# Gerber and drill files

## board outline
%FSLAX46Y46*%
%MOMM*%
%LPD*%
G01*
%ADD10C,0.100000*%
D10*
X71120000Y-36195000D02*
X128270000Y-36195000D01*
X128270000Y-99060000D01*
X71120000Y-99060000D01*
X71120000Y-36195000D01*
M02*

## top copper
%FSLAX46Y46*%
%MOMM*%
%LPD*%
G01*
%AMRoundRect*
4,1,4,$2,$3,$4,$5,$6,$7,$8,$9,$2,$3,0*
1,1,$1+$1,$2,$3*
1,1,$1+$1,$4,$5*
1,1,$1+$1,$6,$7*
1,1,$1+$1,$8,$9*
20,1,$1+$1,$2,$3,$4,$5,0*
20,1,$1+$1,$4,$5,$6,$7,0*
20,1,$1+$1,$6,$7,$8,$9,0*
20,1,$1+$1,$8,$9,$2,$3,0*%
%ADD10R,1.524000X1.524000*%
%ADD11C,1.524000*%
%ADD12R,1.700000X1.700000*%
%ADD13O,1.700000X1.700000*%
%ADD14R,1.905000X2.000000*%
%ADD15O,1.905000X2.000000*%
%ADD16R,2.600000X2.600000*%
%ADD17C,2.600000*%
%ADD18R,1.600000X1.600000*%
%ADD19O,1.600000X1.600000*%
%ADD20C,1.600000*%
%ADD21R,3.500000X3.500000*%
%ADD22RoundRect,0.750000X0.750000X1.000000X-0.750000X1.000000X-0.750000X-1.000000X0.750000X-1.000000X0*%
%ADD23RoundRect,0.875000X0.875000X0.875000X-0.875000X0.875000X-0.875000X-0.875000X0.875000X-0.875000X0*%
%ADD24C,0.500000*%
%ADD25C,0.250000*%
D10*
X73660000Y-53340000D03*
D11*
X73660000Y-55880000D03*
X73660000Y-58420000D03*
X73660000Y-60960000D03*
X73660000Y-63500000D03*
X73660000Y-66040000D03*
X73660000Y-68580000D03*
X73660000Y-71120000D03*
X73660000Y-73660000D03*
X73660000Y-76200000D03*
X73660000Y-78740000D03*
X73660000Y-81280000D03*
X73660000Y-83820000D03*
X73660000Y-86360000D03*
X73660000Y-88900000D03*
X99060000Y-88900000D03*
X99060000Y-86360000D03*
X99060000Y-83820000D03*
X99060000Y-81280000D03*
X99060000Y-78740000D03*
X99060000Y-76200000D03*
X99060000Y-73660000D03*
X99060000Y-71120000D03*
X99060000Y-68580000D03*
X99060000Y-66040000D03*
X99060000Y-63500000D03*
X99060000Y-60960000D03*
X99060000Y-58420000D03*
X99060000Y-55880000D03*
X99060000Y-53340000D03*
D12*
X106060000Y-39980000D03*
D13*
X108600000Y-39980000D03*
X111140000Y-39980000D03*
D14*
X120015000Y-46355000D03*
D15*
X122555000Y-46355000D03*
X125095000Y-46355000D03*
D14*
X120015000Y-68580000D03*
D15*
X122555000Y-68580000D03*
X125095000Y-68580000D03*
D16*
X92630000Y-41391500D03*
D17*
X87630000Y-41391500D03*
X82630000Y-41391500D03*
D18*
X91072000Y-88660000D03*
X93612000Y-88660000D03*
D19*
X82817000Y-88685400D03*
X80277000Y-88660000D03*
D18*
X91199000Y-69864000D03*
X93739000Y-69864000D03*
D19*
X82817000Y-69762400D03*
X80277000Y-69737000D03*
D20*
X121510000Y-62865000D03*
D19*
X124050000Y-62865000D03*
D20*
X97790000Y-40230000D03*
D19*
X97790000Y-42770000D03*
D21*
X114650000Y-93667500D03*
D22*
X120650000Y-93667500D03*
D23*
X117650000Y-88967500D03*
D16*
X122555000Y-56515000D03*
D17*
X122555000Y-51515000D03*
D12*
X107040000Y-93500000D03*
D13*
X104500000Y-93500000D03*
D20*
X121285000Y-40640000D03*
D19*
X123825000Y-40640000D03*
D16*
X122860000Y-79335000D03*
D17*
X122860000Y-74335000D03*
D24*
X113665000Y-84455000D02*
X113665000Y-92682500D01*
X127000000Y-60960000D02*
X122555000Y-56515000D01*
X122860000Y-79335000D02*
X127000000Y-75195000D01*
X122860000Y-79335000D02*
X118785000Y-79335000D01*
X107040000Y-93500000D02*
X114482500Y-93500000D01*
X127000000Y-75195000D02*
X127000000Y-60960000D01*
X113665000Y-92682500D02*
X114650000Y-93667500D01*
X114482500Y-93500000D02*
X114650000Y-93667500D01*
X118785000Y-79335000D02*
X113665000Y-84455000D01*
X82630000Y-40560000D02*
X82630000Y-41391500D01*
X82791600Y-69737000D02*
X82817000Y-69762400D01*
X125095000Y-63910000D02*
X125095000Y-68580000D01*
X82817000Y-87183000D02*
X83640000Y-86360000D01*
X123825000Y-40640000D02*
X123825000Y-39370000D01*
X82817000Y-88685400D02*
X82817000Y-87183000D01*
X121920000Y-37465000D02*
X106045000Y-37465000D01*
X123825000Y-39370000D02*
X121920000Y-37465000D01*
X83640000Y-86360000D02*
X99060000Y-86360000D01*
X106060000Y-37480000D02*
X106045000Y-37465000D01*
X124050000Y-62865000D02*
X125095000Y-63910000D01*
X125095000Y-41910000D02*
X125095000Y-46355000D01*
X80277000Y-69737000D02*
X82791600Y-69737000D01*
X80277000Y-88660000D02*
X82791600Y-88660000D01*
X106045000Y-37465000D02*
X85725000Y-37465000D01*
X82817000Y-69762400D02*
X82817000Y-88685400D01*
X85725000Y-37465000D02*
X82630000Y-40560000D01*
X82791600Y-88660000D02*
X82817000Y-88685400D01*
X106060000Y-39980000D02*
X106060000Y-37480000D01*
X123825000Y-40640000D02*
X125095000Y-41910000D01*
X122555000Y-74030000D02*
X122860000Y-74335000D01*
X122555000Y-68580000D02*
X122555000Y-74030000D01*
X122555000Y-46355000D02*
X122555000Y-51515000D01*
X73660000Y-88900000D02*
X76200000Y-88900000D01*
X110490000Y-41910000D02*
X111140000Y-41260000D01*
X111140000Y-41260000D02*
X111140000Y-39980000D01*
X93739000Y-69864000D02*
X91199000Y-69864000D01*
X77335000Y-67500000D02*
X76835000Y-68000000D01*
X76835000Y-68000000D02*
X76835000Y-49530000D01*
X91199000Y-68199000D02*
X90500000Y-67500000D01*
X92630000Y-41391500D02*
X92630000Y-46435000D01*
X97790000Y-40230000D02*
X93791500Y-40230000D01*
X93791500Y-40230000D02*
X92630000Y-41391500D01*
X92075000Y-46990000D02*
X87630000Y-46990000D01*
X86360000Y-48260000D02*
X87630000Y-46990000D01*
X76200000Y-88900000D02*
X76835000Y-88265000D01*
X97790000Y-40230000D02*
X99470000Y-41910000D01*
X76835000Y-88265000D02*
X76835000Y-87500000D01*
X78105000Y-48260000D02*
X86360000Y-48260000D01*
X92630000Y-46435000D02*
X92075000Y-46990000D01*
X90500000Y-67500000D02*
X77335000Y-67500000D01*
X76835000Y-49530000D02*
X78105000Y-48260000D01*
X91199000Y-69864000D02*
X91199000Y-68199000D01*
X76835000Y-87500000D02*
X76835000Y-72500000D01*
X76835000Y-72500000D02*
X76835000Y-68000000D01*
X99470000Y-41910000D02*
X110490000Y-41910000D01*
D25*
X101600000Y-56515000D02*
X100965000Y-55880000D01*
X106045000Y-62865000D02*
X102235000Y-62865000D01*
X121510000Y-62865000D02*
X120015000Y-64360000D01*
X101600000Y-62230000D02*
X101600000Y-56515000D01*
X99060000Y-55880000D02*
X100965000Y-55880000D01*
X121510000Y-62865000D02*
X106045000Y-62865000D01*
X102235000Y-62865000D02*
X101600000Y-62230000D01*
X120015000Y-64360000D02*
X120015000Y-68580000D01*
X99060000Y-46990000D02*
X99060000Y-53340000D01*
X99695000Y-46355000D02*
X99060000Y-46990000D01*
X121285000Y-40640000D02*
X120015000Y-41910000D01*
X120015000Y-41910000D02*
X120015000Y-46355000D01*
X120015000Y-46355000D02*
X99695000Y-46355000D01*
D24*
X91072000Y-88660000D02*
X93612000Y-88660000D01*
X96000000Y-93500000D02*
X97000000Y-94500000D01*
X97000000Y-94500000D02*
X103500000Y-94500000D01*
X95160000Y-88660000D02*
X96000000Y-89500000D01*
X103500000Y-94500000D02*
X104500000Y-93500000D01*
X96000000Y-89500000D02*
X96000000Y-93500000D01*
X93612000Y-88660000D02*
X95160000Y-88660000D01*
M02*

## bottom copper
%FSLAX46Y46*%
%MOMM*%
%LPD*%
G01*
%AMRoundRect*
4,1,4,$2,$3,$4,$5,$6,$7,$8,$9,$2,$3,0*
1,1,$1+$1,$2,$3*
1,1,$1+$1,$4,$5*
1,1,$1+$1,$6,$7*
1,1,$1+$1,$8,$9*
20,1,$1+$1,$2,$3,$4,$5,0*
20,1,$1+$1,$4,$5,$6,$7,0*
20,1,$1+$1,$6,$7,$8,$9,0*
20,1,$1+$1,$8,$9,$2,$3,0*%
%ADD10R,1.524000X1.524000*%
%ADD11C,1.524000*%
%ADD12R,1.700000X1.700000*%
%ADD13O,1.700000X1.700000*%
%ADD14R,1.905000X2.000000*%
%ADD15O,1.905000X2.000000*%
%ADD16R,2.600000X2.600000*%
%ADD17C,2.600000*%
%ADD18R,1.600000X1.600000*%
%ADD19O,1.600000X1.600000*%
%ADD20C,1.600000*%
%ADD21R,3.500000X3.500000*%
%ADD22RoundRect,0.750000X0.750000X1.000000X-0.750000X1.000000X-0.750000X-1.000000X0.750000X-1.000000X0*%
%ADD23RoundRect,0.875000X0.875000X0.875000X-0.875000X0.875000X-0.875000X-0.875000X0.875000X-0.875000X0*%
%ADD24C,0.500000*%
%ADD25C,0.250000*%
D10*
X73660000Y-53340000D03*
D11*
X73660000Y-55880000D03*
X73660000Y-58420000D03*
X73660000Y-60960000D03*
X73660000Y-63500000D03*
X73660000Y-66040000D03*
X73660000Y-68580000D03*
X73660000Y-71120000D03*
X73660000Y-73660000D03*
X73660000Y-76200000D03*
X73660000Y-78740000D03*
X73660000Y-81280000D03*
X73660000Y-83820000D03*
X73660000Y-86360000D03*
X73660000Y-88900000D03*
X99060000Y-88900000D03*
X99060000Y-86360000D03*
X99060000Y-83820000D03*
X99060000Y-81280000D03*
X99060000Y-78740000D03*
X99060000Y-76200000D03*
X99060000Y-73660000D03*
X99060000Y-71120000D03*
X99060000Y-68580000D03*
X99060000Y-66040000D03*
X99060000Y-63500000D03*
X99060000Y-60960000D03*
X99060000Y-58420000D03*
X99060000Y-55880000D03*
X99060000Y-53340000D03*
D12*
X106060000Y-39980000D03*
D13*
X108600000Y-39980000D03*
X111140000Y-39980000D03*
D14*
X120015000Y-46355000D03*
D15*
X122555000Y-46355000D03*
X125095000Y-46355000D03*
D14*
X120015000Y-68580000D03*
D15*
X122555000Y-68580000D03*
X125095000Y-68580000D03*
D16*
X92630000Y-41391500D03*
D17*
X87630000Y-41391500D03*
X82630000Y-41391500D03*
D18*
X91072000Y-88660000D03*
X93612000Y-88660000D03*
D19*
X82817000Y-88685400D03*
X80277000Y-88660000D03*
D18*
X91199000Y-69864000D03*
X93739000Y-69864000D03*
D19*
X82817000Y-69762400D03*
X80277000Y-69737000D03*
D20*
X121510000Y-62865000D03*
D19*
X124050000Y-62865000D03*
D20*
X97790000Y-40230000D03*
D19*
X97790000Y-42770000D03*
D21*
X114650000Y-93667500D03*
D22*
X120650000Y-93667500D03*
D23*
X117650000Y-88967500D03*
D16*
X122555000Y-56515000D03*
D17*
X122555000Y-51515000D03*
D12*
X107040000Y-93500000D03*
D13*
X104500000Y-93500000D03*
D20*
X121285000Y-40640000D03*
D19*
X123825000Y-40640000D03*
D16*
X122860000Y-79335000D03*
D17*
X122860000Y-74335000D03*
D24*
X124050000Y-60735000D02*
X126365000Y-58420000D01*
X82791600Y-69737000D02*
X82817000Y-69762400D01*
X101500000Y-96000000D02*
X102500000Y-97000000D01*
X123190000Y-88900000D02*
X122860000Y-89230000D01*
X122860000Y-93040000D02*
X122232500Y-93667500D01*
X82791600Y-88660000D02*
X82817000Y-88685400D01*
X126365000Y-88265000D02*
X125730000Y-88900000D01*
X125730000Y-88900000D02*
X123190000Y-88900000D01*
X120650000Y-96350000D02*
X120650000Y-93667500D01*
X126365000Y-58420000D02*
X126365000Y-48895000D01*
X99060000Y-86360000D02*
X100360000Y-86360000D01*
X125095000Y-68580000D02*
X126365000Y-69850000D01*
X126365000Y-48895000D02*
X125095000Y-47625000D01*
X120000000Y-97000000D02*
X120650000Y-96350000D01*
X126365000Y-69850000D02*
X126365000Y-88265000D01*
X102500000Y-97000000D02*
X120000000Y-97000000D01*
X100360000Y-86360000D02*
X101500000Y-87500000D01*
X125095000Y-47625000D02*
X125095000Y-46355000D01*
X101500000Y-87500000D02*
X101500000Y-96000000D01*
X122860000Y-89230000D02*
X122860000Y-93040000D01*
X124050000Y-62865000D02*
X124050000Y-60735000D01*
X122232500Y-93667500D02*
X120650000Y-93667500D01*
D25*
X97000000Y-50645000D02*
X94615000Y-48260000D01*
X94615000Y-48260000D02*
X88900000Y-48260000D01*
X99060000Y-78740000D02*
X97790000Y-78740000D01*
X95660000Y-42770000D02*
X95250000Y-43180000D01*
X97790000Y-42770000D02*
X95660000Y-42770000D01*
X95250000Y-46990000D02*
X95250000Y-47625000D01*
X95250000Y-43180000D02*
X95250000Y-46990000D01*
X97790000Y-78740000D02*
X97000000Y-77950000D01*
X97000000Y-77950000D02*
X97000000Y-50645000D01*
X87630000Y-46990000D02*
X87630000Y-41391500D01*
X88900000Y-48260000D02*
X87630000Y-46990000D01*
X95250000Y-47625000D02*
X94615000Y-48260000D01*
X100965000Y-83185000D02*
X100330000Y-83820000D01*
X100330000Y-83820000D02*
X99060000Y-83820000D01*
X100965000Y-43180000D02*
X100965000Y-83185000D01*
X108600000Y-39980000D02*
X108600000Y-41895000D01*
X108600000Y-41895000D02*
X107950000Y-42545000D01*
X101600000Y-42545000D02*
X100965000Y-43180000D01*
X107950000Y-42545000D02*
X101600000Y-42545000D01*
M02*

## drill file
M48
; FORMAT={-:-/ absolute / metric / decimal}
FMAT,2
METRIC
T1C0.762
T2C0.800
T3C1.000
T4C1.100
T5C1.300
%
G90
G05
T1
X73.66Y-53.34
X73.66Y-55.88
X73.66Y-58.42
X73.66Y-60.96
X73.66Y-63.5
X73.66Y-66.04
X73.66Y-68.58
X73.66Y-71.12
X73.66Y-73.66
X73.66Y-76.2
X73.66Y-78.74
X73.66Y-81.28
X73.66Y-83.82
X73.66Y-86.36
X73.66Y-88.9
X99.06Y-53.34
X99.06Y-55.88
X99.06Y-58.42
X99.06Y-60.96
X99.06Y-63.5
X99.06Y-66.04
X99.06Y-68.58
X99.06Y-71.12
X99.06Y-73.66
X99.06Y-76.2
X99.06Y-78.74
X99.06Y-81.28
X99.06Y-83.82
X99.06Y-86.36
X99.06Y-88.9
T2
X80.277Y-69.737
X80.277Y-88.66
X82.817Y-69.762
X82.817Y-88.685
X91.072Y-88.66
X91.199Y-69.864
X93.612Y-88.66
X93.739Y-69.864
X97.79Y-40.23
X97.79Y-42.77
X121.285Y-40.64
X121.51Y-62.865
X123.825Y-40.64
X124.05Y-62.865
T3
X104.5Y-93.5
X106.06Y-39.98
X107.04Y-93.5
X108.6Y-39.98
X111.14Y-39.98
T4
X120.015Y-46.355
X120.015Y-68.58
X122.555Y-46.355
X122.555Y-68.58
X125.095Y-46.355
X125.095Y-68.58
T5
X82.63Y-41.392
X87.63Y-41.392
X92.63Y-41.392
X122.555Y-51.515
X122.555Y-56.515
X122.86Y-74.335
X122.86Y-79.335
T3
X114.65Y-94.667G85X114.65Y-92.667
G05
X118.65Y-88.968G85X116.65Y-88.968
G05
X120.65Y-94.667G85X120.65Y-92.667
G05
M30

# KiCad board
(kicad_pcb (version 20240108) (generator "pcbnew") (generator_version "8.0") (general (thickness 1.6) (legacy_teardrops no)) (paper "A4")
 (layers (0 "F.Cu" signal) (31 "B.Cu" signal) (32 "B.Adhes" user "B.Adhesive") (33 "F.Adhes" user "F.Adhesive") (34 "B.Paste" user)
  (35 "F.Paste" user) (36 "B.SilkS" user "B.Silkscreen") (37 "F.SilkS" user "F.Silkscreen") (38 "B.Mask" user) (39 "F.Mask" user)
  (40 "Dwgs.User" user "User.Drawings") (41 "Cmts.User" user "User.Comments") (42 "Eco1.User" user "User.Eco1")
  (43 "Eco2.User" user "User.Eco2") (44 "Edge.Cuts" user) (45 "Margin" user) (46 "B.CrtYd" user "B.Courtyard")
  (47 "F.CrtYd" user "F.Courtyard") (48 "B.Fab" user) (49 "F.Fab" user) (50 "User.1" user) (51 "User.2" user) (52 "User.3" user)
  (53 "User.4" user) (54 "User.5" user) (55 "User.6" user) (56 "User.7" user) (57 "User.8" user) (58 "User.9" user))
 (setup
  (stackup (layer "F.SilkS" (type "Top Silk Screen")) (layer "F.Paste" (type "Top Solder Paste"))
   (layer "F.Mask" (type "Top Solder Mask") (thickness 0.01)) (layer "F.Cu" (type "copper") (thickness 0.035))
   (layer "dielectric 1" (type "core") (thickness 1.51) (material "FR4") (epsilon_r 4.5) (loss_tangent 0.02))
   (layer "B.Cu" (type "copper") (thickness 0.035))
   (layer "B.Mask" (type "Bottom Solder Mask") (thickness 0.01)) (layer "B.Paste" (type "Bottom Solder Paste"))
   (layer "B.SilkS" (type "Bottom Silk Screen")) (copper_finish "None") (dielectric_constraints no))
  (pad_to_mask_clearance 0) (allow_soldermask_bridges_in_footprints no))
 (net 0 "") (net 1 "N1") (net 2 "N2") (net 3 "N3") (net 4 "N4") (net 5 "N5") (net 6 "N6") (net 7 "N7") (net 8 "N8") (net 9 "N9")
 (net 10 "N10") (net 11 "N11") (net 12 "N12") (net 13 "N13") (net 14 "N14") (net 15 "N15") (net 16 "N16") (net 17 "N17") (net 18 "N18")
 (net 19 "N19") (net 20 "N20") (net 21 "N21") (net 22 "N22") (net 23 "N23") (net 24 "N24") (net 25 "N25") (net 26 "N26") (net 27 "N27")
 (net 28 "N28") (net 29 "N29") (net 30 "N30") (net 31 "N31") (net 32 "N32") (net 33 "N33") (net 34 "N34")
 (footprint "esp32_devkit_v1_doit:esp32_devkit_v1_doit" (layer "F.Cu") (at 86.36 53.34)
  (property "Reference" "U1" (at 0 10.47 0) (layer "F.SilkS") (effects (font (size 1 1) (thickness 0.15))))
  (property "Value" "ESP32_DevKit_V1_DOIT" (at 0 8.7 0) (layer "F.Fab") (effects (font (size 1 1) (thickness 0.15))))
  (pad "1" thru_hole rect (at -12.7 0) (size 1.524 1.524) (drill 0.762) (layers "*.Cu" "*.Mask") (remove_unused_layers no) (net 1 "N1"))
  (pad "2" thru_hole circle (at -12.7 2.54) (size 1.524 1.524) (drill 0.762) (layers "*.Cu" "*.Mask") (remove_unused_layers no) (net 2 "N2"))
  (pad "3" thru_hole circle (at -12.7 5.08) (size 1.524 1.524) (drill 0.762) (layers "*.Cu" "*.Mask") (remove_unused_layers no) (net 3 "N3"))
  (pad "4" thru_hole circle (at -12.7 7.62) (size 1.524 1.524) (drill 0.762) (layers "*.Cu" "*.Mask") (remove_unused_layers no) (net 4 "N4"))
  (pad "5" thru_hole circle (at -12.7 10.16) (size 1.524 1.524) (drill 0.762) (layers "*.Cu" "*.Mask") (remove_unused_layers no)
   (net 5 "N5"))
  (pad "6" thru_hole circle (at -12.7 12.7) (size 1.524 1.524) (drill 0.762) (layers "*.Cu" "*.Mask") (remove_unused_layers no) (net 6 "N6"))
  (pad "7" thru_hole circle (at -12.7 15.24) (size 1.524 1.524) (drill 0.762) (layers "*.Cu" "*.Mask") (remove_unused_layers no)
   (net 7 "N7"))
  (pad "8" thru_hole circle (at -12.7 17.78) (size 1.524 1.524) (drill 0.762) (layers "*.Cu" "*.Mask") (remove_unused_layers no)
   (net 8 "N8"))
  (pad "9" thru_hole circle (at -12.7 20.32) (size 1.524 1.524) (drill 0.762) (layers "*.Cu" "*.Mask") (remove_unused_layers no)
   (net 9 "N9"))
  (pad "10" thru_hole circle (at -12.7 22.86) (size 1.524 1.524) (drill 0.762) (layers "*.Cu" "*.Mask") (remove_unused_layers no)
   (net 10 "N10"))
  (pad "11" thru_hole circle (at -12.7 25.4) (size 1.524 1.524) (drill 0.762) (layers "*.Cu" "*.Mask") (remove_unused_layers no)
   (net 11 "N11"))
  (pad "12" thru_hole circle (at -12.7 27.94) (size 1.524 1.524) (drill 0.762) (layers "*.Cu" "*.Mask") (remove_unused_layers no)
   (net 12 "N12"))
  (pad "13" thru_hole circle (at -12.7 30.48) (size 1.524 1.524) (drill 0.762) (layers "*.Cu" "*.Mask") (remove_unused_layers no)
   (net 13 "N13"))
  (pad "14" thru_hole circle (at -12.7 33.02) (size 1.524 1.524) (drill 0.762) (layers "*.Cu" "*.Mask") (remove_unused_layers no)
   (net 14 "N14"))
  (pad "15" thru_hole circle (at -12.7 35.56) (size 1.524 1.524) (drill 0.762) (layers "*.Cu" "*.Mask") (remove_unused_layers no)
   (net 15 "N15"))
  (pad "16" thru_hole circle (at 12.7 35.56) (size 1.524 1.524) (drill 0.762) (layers "*.Cu" "*.Mask") (remove_unused_layers no)
   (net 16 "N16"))
  (pad "17" thru_hole circle (at 12.7 33.02) (size 1.524 1.524) (drill 0.762) (layers "*.Cu" "*.Mask") (remove_unused_layers no)
   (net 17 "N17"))
  (pad "18" thru_hole circle (at 12.7 30.48) (size 1.524 1.524) (drill 0.762) (layers "*.Cu" "*.Mask") (remove_unused_layers no)
   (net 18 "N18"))
  (pad "19" thru_hole circle (at 12.7 27.94) (size 1.524 1.524) (drill 0.762) (layers "*.Cu" "*.Mask") (remove_unused_layers no)
   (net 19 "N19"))
  (pad "20" thru_hole circle (at 12.7 25.4) (size 1.524 1.524) (drill 0.762) (layers "*.Cu" "*.Mask") (remove_unused_layers no)
   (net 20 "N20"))
  (pad "21" thru_hole circle (at 12.7 22.86) (size 1.524 1.524) (drill 0.762) (layers "*.Cu" "*.Mask") (remove_unused_layers no)
   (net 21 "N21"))
  (pad "22" thru_hole circle (at 12.7 20.32) (size 1.524 1.524) (drill 0.762) (layers "*.Cu" "*.Mask") (remove_unused_layers no)
   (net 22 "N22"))
  (pad "23" thru_hole circle (at 12.7 17.78) (size 1.524 1.524) (drill 0.762) (layers "*.Cu" "*.Mask") (remove_unused_layers no)
   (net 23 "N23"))
  (pad "24" thru_hole circle (at 12.7 15.24) (size 1.524 1.524) (drill 0.762) (layers "*.Cu" "*.Mask") (remove_unused_layers no)
   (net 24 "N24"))
  (pad "25" thru_hole circle (at 12.7 12.7) (size 1.524 1.524) (drill 0.762) (layers "*.Cu" "*.Mask") (remove_unused_layers no)
   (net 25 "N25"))
  (pad "26" thru_hole circle (at 12.7 10.16) (size 1.524 1.524) (drill 0.762) (layers "*.Cu" "*.Mask") (remove_unused_layers no)
   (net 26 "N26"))
  (pad "27" thru_hole circle (at 12.7 7.62) (size 1.524 1.524) (drill 0.762) (layers "*.Cu" "*.Mask") (remove_unused_layers no)
   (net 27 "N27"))
  (pad "28" thru_hole circle (at 12.7 5.08) (size 1.524 1.524) (drill 0.762) (layers "*.Cu" "*.Mask") (remove_unused_layers no)
   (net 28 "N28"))
  (pad "29" thru_hole circle (at 12.7 2.54) (size 1.524 1.524) (drill 0.762) (layers "*.Cu" "*.Mask") (remove_unused_layers no)
   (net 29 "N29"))
  (pad "30" thru_hole circle (at 12.7 0) (size 1.524 1.524) (drill 0.762) (layers "*.Cu" "*.Mask") (remove_unused_layers no) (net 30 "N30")))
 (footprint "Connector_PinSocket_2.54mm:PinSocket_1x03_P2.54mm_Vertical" (layer "F.Cu") (at 106.06 39.98 90)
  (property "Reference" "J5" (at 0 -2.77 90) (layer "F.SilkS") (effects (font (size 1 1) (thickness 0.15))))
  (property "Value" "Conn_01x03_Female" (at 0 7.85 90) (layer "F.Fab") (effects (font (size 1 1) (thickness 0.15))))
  (pad "1" thru_hole rect (at 0 0 90) (size 1.7 1.7) (drill 1) (layers "*.Cu" "*.Mask") (remove_unused_layers no) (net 17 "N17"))
  (pad "2" thru_hole oval (at 0 2.54 90) (size 1.7 1.7) (drill 1) (layers "*.Cu" "*.Mask") (remove_unused_layers no) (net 18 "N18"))
  (pad "3" thru_hole oval (at 0 5.08 90) (size 1.7 1.7) (drill 1) (layers "*.Cu" "*.Mask") (remove_unused_layers no) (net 15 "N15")))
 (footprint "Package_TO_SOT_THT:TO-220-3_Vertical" (layer "F.Cu") (at 120.015 46.355)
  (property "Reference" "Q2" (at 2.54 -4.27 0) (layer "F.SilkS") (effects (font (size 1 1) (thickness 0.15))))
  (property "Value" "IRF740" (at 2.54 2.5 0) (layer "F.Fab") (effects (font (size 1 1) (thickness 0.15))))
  (pad "1" thru_hole rect (at 0 0) (size 1.905 2) (drill 1.1) (layers "*.Cu" "*.Mask") (remove_unused_layers no) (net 30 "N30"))
  (pad "2" thru_hole oval (at 2.54 0) (size 1.905 2) (drill 1.1) (layers "*.Cu" "*.Mask") (remove_unused_layers no) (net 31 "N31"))
  (pad "3" thru_hole oval (at 5.08 0) (size 1.905 2) (drill 1.1) (layers "*.Cu" "*.Mask") (remove_unused_layers no) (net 17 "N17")))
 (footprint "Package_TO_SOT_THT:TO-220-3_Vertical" (layer "F.Cu") (at 120.015 68.58)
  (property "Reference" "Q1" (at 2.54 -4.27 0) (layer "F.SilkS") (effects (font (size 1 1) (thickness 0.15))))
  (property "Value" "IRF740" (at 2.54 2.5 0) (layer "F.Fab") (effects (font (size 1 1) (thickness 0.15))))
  (pad "1" thru_hole rect (at 0 0) (size 1.905 2) (drill 1.1) (layers "*.Cu" "*.Mask") (remove_unused_layers no) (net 29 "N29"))
  (pad "2" thru_hole oval (at 2.54 0) (size 1.905 2) (drill 1.1) (layers "*.Cu" "*.Mask") (remove_unused_layers no) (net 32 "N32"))
  (pad "3" thru_hole oval (at 5.08 0) (size 1.905 2) (drill 1.1) (layers "*.Cu" "*.Mask") (remove_unused_layers no) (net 17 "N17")))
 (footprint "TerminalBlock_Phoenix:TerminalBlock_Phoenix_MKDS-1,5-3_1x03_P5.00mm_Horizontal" (layer "F.Cu") (at 92.63 41.3915 180)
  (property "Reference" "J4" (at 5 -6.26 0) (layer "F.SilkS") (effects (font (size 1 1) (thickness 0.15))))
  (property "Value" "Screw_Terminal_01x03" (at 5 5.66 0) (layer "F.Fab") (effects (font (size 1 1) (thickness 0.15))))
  (pad "1" thru_hole rect (at 0 0 180) (size 2.6 2.6) (drill 1.3) (layers "*.Cu" "*.Mask") (remove_unused_layers no) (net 15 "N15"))
  (pad "2" thru_hole circle (at 5 0 180) (size 2.6 2.6) (drill 1.3) (layers "*.Cu" "*.Mask") (remove_unused_layers no) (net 20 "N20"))
  (pad "3" thru_hole circle (at 10 0 180) (size 2.6 2.6) (drill 1.3) (layers "*.Cu" "*.Mask") (remove_unused_layers no) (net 17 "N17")))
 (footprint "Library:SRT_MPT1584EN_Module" (layer "F.Cu") (at 86.5 78.5 90)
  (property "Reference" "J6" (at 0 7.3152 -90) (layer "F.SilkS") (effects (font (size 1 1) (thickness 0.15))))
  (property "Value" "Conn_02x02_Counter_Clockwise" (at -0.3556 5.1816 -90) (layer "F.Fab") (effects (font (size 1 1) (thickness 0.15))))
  (pad "1" thru_hole rect (at -10.16 4.572 180) (size 1.6 1.6) (drill 0.8) (layers "*.Cu" "B.Mask") (remove_unused_layers no) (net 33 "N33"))
  (pad "1" thru_hole rect (at -10.16 7.112 180) (size 1.6 1.6) (drill 0.8) (layers "*.Cu" "B.Mask") (remove_unused_layers no) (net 33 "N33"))
  (pad "2" thru_hole oval (at -10.1854 -3.683 180) (size 1.6 1.6) (drill 0.8) (layers "*.Cu" "B.Mask") (remove_unused_layers no)
   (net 17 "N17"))
  (pad "2" thru_hole oval (at -10.16 -6.223 180) (size 1.6 1.6) (drill 0.8) (layers "*.Cu" "B.Mask") (remove_unused_layers no)
   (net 17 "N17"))
  (pad "3" thru_hole rect (at 8.636 4.699 180) (size 1.6 1.6) (drill 0.8) (layers "*.Cu" "B.Mask") (remove_unused_layers no) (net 15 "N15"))
  (pad "3" thru_hole rect (at 8.636 7.239 180) (size 1.6 1.6) (drill 0.8) (layers "*.Cu" "B.Mask") (remove_unused_layers no) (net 15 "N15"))
  (pad "4" thru_hole oval (at 8.7376 -3.683 180) (size 1.6 1.6) (drill 0.8) (layers "*.Cu" "B.Mask") (remove_unused_layers no)
   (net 17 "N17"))
  (pad "4" thru_hole oval (at 8.763 -6.223 180) (size 1.6 1.6) (drill 0.8) (layers "*.Cu" "B.Mask") (remove_unused_layers no) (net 17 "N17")))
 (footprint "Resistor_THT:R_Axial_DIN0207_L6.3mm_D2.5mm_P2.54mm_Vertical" (layer "F.Cu") (at 121.51 62.865)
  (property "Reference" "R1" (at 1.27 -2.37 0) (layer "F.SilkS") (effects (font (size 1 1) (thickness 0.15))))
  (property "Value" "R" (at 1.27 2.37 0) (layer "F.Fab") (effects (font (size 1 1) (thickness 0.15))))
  (pad "1" thru_hole circle (at 0 0) (size 1.6 1.6) (drill 0.8) (layers "*.Cu" "*.Mask") (remove_unused_layers no) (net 29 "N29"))
  (pad "2" thru_hole oval (at 2.54 0) (size 1.6 1.6) (drill 0.8) (layers "*.Cu" "*.Mask") (remove_unused_layers no) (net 17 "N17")))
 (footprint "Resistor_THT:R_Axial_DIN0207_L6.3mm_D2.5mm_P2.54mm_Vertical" (layer "F.Cu") (at 97.79 40.23 -90)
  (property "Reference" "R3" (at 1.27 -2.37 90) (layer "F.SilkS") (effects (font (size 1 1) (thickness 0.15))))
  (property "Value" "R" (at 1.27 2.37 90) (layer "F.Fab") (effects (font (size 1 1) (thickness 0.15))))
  (pad "1" thru_hole circle (at 0 0 270) (size 1.6 1.6) (drill 0.8) (layers "*.Cu" "*.Mask") (remove_unused_layers no) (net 15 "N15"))
  (pad "2" thru_hole oval (at 2.54 0 270) (size 1.6 1.6) (drill 0.8) (layers "*.Cu" "*.Mask") (remove_unused_layers no) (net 20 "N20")))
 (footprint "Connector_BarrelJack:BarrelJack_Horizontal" (layer "F.Cu") (at 114.65 93.6675 180)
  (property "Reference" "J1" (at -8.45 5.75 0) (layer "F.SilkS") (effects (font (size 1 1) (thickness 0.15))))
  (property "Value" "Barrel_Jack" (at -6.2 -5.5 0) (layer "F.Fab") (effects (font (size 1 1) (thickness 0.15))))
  (pad "1" thru_hole rect (at 0 0 180) (size 3.5 3.5) (drill oval 1 3) (layers "*.Cu" "*.Mask") (remove_unused_layers no) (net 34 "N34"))
  (pad "2" thru_hole roundrect (at -6 0 180) (size 3 3.5) (drill oval 1 3) (layers "*.Cu" "*.Mask") (remove_unused_layers no)
   (roundrect_rratio 0.25) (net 17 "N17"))
  (pad "3" thru_hole roundrect (at -3 4.7 180) (size 3.5 3.5) (drill oval 3 1) (layers "*.Cu" "*.Mask") (remove_unused_layers no)
   (roundrect_rratio 0.25)))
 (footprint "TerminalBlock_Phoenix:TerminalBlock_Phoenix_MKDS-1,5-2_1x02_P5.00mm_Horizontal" (layer "F.Cu") (at 122.555 56.515 90)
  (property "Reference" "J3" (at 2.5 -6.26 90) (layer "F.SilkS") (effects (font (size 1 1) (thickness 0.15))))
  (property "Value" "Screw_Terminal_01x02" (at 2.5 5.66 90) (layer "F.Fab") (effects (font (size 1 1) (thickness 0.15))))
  (pad "1" thru_hole rect (at 0 0 90) (size 2.6 2.6) (drill 1.3) (layers "*.Cu" "*.Mask") (remove_unused_layers no) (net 34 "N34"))
  (pad "2" thru_hole circle (at 5 0 90) (size 2.6 2.6) (drill 1.3) (layers "*.Cu" "*.Mask") (remove_unused_layers no) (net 31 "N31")))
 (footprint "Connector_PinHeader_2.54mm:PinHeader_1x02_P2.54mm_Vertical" (layer "F.Cu") (at 107.04 93.5 -90)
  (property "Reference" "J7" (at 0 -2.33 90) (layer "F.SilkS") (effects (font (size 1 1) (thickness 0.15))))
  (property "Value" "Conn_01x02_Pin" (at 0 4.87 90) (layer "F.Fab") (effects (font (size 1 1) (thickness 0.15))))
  (pad "1" thru_hole rect (at 0 0 270) (size 1.7 1.7) (drill 1) (layers "*.Cu" "*.Mask") (remove_unused_layers no) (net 34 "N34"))
  (pad "2" thru_hole oval (at 0 2.54 270) (size 1.7 1.7) (drill 1) (layers "*.Cu" "*.Mask") (remove_unused_layers no) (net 33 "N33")))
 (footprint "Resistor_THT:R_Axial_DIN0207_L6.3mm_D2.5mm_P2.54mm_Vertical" (layer "F.Cu") (at 121.285 40.64)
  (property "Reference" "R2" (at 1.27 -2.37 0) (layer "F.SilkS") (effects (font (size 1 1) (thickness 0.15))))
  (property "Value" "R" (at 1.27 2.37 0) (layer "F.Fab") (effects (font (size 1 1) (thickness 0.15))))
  (pad "1" thru_hole circle (at 0 0) (size 1.6 1.6) (drill 0.8) (layers "*.Cu" "*.Mask") (remove_unused_layers no) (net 30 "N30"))
  (pad "2" thru_hole oval (at 2.54 0) (size 1.6 1.6) (drill 0.8) (layers "*.Cu" "*.Mask") (remove_unused_layers no) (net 17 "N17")))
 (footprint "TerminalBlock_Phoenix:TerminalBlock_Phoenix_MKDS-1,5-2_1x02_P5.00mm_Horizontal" (layer "F.Cu") (at 122.86 79.335 90)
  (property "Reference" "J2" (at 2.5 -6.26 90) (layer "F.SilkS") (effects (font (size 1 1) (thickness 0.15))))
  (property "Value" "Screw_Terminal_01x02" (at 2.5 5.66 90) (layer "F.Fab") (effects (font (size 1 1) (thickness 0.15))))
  (pad "1" thru_hole rect (at 0 0 90) (size 2.6 2.6) (drill 1.3) (layers "*.Cu" "*.Mask") (remove_unused_layers no) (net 34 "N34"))
  (pad "2" thru_hole circle (at 5 0 90) (size 2.6 2.6) (drill 1.3) (layers "*.Cu" "*.Mask") (remove_unused_layers no) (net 32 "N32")))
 (gr_rect (start 71.12 36.195) (end 128.27 99.06) (stroke (width 0.1) (type solid)) (fill none) (layer "Edge.Cuts"))
 (segment (start 113.665 84.455) (end 113.665 92.6825) (width 0.5) (layer "F.Cu") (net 34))
 (segment (start 127 60.96) (end 122.555 56.515) (width 0.5) (layer "F.Cu") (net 34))
 (segment (start 122.86 79.335) (end 127 75.195) (width 0.5) (layer "F.Cu") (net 34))
 (segment (start 122.86 79.335) (end 118.785 79.335) (width 0.5) (layer "F.Cu") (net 34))
 (segment (start 107.04 93.5) (end 114.4825 93.5) (width 0.5) (layer "F.Cu") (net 34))
 (segment (start 127 75.195) (end 127 60.96) (width 0.5) (layer "F.Cu") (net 34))
 (segment (start 113.665 92.6825) (end 114.65 93.6675) (width 0.5) (layer "F.Cu") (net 34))
 (segment (start 114.4825 93.5) (end 114.65 93.6675) (width 0.5) (layer "F.Cu") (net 34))
 (segment (start 118.785 79.335) (end 113.665 84.455) (width 0.5) (layer "F.Cu") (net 34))
 (segment (start 82.63 40.56) (end 82.63 41.3915) (width 0.5) (layer "F.Cu") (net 17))
 (segment (start 82.7916 69.737) (end 82.817 69.7624) (width 0.5) (layer "F.Cu") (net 17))
 (segment (start 125.095 63.91) (end 125.095 68.58) (width 0.5) (layer "F.Cu") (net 17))
 (segment (start 82.817 87.183) (end 83.64 86.36) (width 0.5) (layer "F.Cu") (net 17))
 (segment (start 123.825 40.64) (end 123.825 39.37) (width 0.5) (layer "F.Cu") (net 17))
 (segment (start 82.817 88.6854) (end 82.817 87.183) (width 0.5) (layer "F.Cu") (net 17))
 (segment (start 121.92 37.465) (end 106.045 37.465) (width 0.5) (layer "F.Cu") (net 17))
 (segment (start 123.825 39.37) (end 121.92 37.465) (width 0.5) (layer "F.Cu") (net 17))
 (segment (start 83.64 86.36) (end 99.06 86.36) (width 0.5) (layer "F.Cu") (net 17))
 (segment (start 106.06 37.48) (end 106.045 37.465) (width 0.5) (layer "F.Cu") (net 17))
 (segment (start 124.05 62.865) (end 125.095 63.91) (width 0.5) (layer "F.Cu") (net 17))
 (segment (start 125.095 41.91) (end 125.095 46.355) (width 0.5) (layer "F.Cu") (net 17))
 (segment (start 80.277 69.737) (end 82.7916 69.737) (width 0.5) (layer "F.Cu") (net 17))
 (segment (start 80.277 88.66) (end 82.7916 88.66) (width 0.5) (layer "F.Cu") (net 17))
 (segment (start 106.045 37.465) (end 85.725 37.465) (width 0.5) (layer "F.Cu") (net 17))
 (segment (start 82.817 69.7624) (end 82.817 88.6854) (width 0.5) (layer "F.Cu") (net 17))
 (segment (start 85.725 37.465) (end 82.63 40.56) (width 0.5) (layer "F.Cu") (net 17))
 (segment (start 82.7916 88.66) (end 82.817 88.6854) (width 0.5) (layer "F.Cu") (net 17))
 (segment (start 106.06 39.98) (end 106.06 37.48) (width 0.5) (layer "F.Cu") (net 17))
 (segment (start 123.825 40.64) (end 125.095 41.91) (width 0.5) (layer "F.Cu") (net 17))
 (segment (start 124.05 60.735) (end 126.365 58.42) (width 0.5) (layer "B.Cu") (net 17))
 (segment (start 82.7916 69.737) (end 82.817 69.7624) (width 0.5) (layer "B.Cu") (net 17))
 (segment (start 101.5 96) (end 102.5 97) (width 0.5) (layer "B.Cu") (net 17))
 (segment (start 123.19 88.9) (end 122.86 89.23) (width 0.5) (layer "B.Cu") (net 17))
 (segment (start 122.86 93.04) (end 122.2325 93.6675) (width 0.5) (layer "B.Cu") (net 17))
 (segment (start 82.7916 88.66) (end 82.817 88.6854) (width 0.5) (layer "B.Cu") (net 17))
 (segment (start 126.365 88.265) (end 125.73 88.9) (width 0.5) (layer "B.Cu") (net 17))
 (segment (start 125.73 88.9) (end 123.19 88.9) (width 0.5) (layer "B.Cu") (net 17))
 (segment (start 120.65 96.35) (end 120.65 93.6675) (width 0.5) (layer "B.Cu") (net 17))
 (segment (start 126.365 58.42) (end 126.365 48.895) (width 0.5) (layer "B.Cu") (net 17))
 (segment (start 99.06 86.36) (end 100.36 86.36) (width 0.5) (layer "B.Cu") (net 17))
 (segment (start 125.095 68.58) (end 126.365 69.85) (width 0.5) (layer "B.Cu") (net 17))
 (segment (start 126.365 48.895) (end 125.095 47.625) (width 0.5) (layer "B.Cu") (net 17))
 (segment (start 120 97) (end 120.65 96.35) (width 0.5) (layer "B.Cu") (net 17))
 (segment (start 126.365 69.85) (end 126.365 88.265) (width 0.5) (layer "B.Cu") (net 17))
 (segment (start 102.5 97) (end 120 97) (width 0.5) (layer "B.Cu") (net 17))
 (segment (start 100.36 86.36) (end 101.5 87.5) (width 0.5) (layer "B.Cu") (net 17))
 (segment (start 125.095 47.625) (end 125.095 46.355) (width 0.5) (layer "B.Cu") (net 17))
 (segment (start 101.5 87.5) (end 101.5 96) (width 0.5) (layer "B.Cu") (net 17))
 (segment (start 122.86 89.23) (end 122.86 93.04) (width 0.5) (layer "B.Cu") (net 17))
 (segment (start 124.05 62.865) (end 124.05 60.735) (width 0.5) (layer "B.Cu") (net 17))
 (segment (start 122.2325 93.6675) (end 120.65 93.6675) (width 0.5) (layer "B.Cu") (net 17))
 (segment (start 122.555 74.03) (end 122.86 74.335) (width 0.5) (layer "F.Cu") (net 32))
 (segment (start 122.555 68.58) (end 122.555 74.03) (width 0.5) (layer "F.Cu") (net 32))
 (segment (start 122.555 46.355) (end 122.555 51.515) (width 0.5) (layer "F.Cu") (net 31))
 (segment (start 97 50.645) (end 94.615 48.26) (width 0.25) (layer "B.Cu") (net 20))
 (segment (start 94.615 48.26) (end 88.9 48.26) (width 0.25) (layer "B.Cu") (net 20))
 (segment (start 99.06 78.74) (end 97.79 78.74) (width 0.25) (layer "B.Cu") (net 20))
 (segment (start 95.66 42.77) (end 95.25 43.18) (width 0.25) (layer "B.Cu") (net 20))
 (segment (start 97.79 42.77) (end 95.66 42.77) (width 0.25) (layer "B.Cu") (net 20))
 (segment (start 95.25 46.99) (end 95.25 47.625) (width 0.25) (layer "B.Cu") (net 20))
 (segment (start 95.25 43.18) (end 95.25 46.99) (width 0.25) (layer "B.Cu") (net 20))
 (segment (start 97.79 78.74) (end 97 77.95) (width 0.25) (layer "B.Cu") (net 20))
 (segment (start 97 77.95) (end 97 50.645) (width 0.25) (layer "B.Cu") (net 20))
 (segment (start 87.63 46.99) (end 87.63 41.3915) (width 0.25) (layer "B.Cu") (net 20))
 (segment (start 88.9 48.26) (end 87.63 46.99) (width 0.25) (layer "B.Cu") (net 20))
 (segment (start 95.25 47.625) (end 94.615 48.26) (width 0.25) (layer "B.Cu") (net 20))
 (segment (start 73.66 88.9) (end 76.2 88.9) (width 0.5) (layer "F.Cu") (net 15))
 (segment (start 110.49 41.91) (end 111.14 41.26) (width 0.5) (layer "F.Cu") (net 15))
 (segment (start 111.14 41.26) (end 111.14 39.98) (width 0.5) (layer "F.Cu") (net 15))
 (segment (start 93.739 69.864) (end 91.199 69.864) (width 0.5) (layer "F.Cu") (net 15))
 (segment (start 77.335 67.5) (end 76.835 68) (width 0.5) (layer "F.Cu") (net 15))
 (segment (start 76.835 68) (end 76.835 49.53) (width 0.5) (layer "F.Cu") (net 15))
 (segment (start 91.199 68.199) (end 90.5 67.5) (width 0.5) (layer "F.Cu") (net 15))
 (segment (start 92.63 41.3915) (end 92.63 46.435) (width 0.5) (layer "F.Cu") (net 15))
 (segment (start 97.79 40.23) (end 93.7915 40.23) (width 0.5) (layer "F.Cu") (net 15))
 (segment (start 93.7915 40.23) (end 92.63 41.3915) (width 0.5) (layer "F.Cu") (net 15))
 (segment (start 92.075 46.99) (end 87.63 46.99) (width 0.5) (layer "F.Cu") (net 15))
 (segment (start 86.36 48.26) (end 87.63 46.99) (width 0.5) (layer "F.Cu") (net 15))
 (segment (start 76.2 88.9) (end 76.835 88.265) (width 0.5) (layer "F.Cu") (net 15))
 (segment (start 97.79 40.23) (end 99.47 41.91) (width 0.5) (layer "F.Cu") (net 15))
 (segment (start 76.835 88.265) (end 76.835 87.5) (width 0.5) (layer "F.Cu") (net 15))
 (segment (start 78.105 48.26) (end 86.36 48.26) (width 0.5) (layer "F.Cu") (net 15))
 (segment (start 92.63 46.435) (end 92.075 46.99) (width 0.5) (layer "F.Cu") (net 15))
 (segment (start 90.5 67.5) (end 77.335 67.5) (width 0.5) (layer "F.Cu") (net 15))
 (segment (start 76.835 49.53) (end 78.105 48.26) (width 0.5) (layer "F.Cu") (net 15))
 (segment (start 91.199 69.864) (end 91.199 68.199) (width 0.5) (layer "F.Cu") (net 15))
 (segment (start 76.835 87.5) (end 76.835 72.5) (width 0.5) (layer "F.Cu") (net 15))
 (segment (start 76.835 72.5) (end 76.835 68) (width 0.5) (layer "F.Cu") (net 15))
 (segment (start 99.47 41.91) (end 110.49 41.91) (width 0.5) (layer "F.Cu") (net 15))
 (segment (start 100.965 83.185) (end 100.33 83.82) (width 0.25) (layer "B.Cu") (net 18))
 (segment (start 100.33 83.82) (end 99.06 83.82) (width 0.25) (layer "B.Cu") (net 18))
 (segment (start 100.965 43.18) (end 100.965 83.185) (width 0.25) (layer "B.Cu") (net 18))
 (segment (start 108.6 39.98) (end 108.6 41.895) (width 0.25) (layer "B.Cu") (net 18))
 (segment (start 108.6 41.895) (end 107.95 42.545) (width 0.25) (layer "B.Cu") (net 18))
 (segment (start 101.6 42.545) (end 100.965 43.18) (width 0.25) (layer "B.Cu") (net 18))
 (segment (start 107.95 42.545) (end 101.6 42.545) (width 0.25) (layer "B.Cu") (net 18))
 (segment (start 101.6 56.515) (end 100.965 55.88) (width 0.25) (layer "F.Cu") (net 29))
 (segment (start 106.045 62.865) (end 102.235 62.865) (width 0.25) (layer "F.Cu") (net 29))
 (segment (start 121.51 62.865) (end 120.015 64.36) (width 0.25) (layer "F.Cu") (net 29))
 (segment (start 101.6 62.23) (end 101.6 56.515) (width 0.25) (layer "F.Cu") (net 29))
 (segment (start 99.06 55.88) (end 100.965 55.88) (width 0.25) (layer "F.Cu") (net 29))
 (segment (start 121.51 62.865) (end 106.045 62.865) (width 0.25) (layer "F.Cu") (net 29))
 (segment (start 102.235 62.865) (end 101.6 62.23) (width 0.25) (layer "F.Cu") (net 29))
 (segment (start 120.015 64.36) (end 120.015 68.58) (width 0.25) (layer "F.Cu") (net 29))
 (segment (start 99.06 46.99) (end 99.06 53.34) (width 0.25) (layer "F.Cu") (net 30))
 (segment (start 99.695 46.355) (end 99.06 46.99) (width 0.25) (layer "F.Cu") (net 30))
 (segment (start 121.285 40.64) (end 120.015 41.91) (width 0.25) (layer "F.Cu") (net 30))
 (segment (start 120.015 41.91) (end 120.015 46.355) (width 0.25) (layer "F.Cu") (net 30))
 (segment (start 120.015 46.355) (end 99.695 46.355) (width 0.25) (layer "F.Cu") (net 30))
 (segment (start 91.072 88.66) (end 93.612 88.66) (width 0.5) (layer "F.Cu") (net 33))
 (segment (start 96 93.5) (end 97 94.5) (width 0.5) (layer "F.Cu") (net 33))
 (segment (start 97 94.5) (end 103.5 94.5) (width 0.5) (layer "F.Cu") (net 33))
 (segment (start 95.16 88.66) (end 96 89.5) (width 0.5) (layer "F.Cu") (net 33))
 (segment (start 103.5 94.5) (end 104.5 93.5) (width 0.5) (layer "F.Cu") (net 33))
 (segment (start 96 89.5) (end 96 93.5) (width 0.5) (layer "F.Cu") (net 33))
 (segment (start 93.612 88.66) (end 95.16 88.66) (width 0.5) (layer "F.Cu") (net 33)))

